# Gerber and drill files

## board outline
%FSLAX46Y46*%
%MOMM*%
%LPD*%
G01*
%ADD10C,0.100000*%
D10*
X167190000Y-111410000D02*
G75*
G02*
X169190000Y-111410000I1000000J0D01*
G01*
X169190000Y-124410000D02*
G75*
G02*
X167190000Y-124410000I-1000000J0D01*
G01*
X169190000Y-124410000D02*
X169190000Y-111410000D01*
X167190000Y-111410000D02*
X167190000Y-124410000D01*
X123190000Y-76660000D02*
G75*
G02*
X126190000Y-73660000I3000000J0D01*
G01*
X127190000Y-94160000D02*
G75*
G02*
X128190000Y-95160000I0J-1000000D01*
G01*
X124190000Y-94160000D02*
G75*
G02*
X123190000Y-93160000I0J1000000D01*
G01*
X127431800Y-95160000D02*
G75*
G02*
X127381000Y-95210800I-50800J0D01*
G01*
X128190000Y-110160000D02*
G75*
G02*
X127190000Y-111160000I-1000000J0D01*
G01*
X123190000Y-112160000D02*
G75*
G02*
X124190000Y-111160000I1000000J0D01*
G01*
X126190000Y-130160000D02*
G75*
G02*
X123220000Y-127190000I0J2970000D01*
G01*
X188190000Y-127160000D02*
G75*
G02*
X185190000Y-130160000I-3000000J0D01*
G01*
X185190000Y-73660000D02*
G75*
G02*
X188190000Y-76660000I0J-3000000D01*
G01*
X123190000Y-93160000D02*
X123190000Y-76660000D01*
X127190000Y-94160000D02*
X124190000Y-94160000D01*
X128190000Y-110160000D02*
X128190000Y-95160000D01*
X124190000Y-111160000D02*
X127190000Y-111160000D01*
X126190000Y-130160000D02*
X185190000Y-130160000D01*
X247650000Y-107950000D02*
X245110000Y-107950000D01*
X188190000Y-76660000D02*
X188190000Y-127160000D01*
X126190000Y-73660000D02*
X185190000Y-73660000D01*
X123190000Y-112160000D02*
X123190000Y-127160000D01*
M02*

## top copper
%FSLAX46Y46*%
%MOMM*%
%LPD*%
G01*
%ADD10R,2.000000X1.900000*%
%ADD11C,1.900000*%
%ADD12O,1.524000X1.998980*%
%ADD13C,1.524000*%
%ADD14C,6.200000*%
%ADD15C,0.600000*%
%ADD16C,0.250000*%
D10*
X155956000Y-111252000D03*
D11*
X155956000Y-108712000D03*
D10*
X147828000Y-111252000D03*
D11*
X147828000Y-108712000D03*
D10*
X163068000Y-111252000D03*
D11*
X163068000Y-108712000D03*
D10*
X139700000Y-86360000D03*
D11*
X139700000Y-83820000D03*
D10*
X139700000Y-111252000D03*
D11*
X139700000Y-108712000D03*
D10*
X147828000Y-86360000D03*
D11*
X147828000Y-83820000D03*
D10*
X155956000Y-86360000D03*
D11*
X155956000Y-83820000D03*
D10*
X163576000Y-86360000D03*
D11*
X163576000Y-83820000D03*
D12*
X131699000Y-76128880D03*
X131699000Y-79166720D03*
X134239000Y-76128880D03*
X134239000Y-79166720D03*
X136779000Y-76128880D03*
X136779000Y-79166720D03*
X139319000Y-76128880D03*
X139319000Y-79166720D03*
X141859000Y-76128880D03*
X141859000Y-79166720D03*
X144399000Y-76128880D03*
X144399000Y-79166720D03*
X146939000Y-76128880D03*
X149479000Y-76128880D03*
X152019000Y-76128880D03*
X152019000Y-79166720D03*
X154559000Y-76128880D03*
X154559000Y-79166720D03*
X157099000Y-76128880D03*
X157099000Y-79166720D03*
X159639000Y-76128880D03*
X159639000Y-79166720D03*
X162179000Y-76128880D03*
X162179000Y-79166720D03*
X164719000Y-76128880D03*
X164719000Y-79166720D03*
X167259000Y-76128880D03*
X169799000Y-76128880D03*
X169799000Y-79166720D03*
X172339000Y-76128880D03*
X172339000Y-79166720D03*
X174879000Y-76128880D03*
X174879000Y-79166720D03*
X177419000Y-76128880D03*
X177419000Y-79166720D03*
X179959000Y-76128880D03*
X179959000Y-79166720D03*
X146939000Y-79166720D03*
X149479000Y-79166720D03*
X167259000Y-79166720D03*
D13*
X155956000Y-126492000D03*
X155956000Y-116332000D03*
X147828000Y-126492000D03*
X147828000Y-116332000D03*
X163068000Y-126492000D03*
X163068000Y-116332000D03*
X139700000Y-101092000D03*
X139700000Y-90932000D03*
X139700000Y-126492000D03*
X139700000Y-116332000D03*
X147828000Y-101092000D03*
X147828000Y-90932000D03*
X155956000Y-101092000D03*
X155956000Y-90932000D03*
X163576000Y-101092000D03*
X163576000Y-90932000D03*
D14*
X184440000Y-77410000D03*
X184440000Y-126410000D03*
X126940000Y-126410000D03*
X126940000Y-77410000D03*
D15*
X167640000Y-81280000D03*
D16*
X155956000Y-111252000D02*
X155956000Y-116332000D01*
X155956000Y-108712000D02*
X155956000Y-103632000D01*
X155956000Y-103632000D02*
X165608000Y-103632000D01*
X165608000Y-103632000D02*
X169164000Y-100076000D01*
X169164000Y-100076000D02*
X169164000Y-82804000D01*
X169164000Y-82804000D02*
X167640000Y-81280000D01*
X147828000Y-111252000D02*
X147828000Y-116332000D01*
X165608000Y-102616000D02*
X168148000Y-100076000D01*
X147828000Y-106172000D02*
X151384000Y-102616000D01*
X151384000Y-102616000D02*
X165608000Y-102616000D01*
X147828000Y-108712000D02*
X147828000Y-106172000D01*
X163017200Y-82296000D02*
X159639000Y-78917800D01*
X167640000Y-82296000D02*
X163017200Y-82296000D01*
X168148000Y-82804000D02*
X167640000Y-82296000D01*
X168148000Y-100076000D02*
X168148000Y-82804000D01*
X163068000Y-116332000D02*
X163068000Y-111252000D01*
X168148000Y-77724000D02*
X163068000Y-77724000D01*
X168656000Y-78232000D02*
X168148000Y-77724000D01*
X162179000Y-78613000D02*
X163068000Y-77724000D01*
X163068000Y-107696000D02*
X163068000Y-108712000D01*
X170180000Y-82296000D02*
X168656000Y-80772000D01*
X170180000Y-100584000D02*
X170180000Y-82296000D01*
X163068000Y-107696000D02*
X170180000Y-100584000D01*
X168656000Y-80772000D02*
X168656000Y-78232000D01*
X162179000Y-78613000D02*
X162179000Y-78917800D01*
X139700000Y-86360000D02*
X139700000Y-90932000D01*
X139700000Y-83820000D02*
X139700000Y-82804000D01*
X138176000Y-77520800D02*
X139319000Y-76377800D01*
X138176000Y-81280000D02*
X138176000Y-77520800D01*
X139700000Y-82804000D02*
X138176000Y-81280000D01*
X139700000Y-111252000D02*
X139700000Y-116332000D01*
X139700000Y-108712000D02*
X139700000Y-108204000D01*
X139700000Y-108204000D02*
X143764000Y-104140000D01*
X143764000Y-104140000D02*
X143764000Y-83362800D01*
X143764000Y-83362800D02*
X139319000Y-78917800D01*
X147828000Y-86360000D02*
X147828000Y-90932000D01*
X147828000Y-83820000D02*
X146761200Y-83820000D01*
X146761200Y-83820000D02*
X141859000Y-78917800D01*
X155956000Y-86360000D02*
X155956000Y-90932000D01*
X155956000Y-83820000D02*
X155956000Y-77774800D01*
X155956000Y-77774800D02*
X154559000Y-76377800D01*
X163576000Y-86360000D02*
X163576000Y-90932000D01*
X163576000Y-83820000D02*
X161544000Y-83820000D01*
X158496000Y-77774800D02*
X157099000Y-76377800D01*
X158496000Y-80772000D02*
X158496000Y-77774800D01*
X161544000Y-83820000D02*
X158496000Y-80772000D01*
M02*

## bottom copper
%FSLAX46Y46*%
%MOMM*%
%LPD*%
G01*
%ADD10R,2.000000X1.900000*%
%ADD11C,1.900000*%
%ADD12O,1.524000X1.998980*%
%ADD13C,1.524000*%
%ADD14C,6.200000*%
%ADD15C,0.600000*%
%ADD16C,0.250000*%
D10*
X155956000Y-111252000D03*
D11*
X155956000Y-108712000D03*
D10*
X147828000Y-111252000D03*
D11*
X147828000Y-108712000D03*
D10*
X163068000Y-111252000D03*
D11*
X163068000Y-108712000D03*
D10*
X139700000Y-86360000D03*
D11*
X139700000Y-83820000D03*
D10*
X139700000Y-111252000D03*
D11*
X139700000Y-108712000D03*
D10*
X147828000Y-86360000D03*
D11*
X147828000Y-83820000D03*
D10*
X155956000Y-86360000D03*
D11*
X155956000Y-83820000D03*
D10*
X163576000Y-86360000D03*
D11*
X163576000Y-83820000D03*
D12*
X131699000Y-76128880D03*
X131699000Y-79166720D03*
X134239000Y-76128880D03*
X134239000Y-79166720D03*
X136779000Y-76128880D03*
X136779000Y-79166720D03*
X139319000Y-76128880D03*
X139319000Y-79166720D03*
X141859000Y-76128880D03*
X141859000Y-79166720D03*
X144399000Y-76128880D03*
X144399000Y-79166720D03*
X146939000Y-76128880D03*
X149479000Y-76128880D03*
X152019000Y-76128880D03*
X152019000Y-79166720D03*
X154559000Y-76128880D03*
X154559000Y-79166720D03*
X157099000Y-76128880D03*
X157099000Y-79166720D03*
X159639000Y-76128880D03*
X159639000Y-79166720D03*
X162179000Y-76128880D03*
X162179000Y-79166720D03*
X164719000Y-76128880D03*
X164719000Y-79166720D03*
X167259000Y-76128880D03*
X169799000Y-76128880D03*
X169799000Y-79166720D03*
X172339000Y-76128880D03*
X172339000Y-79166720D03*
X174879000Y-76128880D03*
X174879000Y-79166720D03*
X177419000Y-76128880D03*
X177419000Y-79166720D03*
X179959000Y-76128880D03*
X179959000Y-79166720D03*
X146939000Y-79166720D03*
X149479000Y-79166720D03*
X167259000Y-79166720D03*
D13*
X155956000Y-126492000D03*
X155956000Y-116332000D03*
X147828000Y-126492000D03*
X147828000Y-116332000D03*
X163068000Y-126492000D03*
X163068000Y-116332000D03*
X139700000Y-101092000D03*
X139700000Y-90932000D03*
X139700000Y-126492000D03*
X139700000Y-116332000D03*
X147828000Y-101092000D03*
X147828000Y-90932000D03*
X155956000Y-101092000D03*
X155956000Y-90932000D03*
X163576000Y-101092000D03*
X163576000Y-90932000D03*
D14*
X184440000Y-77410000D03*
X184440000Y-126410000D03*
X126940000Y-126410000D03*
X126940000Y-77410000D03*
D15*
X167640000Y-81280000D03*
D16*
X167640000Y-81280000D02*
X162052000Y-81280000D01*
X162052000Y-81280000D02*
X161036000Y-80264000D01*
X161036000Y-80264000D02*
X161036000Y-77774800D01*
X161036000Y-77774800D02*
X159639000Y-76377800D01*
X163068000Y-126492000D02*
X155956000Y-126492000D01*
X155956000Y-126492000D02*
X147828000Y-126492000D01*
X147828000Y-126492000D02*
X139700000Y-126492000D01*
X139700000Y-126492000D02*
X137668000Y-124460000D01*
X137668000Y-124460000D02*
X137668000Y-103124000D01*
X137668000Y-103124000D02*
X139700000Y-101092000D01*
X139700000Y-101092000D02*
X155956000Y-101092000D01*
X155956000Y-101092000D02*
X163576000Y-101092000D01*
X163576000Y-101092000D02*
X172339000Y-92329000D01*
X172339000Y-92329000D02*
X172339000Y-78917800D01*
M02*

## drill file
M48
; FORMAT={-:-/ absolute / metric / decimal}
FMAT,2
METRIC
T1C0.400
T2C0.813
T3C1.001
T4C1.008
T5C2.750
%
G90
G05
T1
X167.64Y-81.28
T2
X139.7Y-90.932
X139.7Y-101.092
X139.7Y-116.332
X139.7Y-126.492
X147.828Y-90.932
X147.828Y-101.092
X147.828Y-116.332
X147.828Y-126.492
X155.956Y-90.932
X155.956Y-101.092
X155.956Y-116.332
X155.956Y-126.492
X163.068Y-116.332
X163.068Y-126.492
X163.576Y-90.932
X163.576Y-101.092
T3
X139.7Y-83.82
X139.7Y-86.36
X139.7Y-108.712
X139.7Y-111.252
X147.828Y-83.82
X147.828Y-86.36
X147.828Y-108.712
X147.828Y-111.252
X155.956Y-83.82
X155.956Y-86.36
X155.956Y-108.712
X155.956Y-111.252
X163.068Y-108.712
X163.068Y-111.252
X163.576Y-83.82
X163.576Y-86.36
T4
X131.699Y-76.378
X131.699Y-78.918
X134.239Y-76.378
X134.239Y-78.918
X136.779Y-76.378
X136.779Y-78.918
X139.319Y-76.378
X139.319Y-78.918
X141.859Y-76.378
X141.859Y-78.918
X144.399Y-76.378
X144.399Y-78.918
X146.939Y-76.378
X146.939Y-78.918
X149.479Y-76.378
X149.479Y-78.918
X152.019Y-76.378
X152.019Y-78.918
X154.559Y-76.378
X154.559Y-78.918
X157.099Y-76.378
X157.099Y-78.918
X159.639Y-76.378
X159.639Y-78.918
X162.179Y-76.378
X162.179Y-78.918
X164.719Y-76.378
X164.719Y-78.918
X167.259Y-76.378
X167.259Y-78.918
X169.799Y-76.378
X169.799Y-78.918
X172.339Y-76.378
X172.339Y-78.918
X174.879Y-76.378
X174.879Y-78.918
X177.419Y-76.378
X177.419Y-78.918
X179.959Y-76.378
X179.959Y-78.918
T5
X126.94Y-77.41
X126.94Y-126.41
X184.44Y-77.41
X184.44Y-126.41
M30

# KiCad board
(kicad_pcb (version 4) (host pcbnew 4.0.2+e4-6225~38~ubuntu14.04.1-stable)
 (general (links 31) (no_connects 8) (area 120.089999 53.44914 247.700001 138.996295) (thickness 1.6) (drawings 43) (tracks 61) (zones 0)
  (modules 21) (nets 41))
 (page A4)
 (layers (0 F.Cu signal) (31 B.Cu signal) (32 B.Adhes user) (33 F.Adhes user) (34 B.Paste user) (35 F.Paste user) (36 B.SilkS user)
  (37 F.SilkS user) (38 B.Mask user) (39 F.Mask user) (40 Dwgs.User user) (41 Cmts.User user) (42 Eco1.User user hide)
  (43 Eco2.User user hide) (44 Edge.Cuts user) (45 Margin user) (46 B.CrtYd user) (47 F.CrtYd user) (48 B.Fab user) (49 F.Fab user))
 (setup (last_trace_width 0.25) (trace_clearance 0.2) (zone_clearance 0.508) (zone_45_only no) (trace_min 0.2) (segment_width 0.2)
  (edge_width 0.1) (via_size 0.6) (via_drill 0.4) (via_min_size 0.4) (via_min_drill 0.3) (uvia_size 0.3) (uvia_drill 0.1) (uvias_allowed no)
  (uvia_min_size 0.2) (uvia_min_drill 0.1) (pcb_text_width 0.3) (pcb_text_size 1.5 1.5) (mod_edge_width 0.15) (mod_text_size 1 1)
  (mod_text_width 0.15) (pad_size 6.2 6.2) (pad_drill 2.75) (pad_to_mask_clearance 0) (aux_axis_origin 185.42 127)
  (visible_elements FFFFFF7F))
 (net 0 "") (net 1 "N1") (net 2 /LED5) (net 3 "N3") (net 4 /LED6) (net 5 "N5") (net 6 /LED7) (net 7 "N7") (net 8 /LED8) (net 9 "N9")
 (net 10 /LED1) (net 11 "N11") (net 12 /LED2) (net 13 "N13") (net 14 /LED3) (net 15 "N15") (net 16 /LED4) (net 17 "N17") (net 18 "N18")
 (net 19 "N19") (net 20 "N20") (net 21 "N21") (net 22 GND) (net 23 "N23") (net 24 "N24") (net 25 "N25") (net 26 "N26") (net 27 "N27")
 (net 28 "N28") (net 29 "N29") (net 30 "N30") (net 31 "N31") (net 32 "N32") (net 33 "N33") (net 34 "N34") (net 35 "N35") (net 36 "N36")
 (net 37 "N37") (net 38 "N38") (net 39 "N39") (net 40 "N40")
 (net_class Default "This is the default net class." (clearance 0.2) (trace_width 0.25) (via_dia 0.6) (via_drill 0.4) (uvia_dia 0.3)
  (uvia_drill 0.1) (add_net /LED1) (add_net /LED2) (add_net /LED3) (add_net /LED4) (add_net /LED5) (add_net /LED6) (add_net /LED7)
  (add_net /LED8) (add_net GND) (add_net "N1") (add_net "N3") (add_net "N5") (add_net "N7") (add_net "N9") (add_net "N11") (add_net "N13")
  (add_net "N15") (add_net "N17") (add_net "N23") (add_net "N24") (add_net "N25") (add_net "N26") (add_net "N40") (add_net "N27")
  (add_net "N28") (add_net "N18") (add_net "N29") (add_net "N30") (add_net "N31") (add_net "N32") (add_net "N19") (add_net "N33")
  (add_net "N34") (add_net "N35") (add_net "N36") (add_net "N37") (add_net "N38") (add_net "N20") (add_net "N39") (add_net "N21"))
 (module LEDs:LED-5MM (layer F.Cu) (at 155.956 111.252 90)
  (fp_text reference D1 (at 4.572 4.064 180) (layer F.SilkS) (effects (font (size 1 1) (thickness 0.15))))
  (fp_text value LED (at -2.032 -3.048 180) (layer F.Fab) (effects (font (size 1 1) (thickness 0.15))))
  (pad 1 thru_hole rect (at 0 0 180) (size 2 1.9) (drill 1.00076) (layers *.Cu *.Mask F.SilkS) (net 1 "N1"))
  (pad 2 thru_hole circle (at 2.54 0 90) (size 1.9 1.9) (drill 1.00076) (layers *.Cu *.Mask F.SilkS) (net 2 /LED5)))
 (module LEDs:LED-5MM (layer F.Cu) (at 147.828 111.252 90)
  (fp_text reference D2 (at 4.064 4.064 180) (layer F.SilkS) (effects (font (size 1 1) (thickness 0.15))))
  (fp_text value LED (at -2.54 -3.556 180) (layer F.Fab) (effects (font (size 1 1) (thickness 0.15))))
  (pad 1 thru_hole rect (at 0 0 180) (size 2 1.9) (drill 1.00076) (layers *.Cu *.Mask F.SilkS) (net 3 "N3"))
  (pad 2 thru_hole circle (at 2.54 0 90) (size 1.9 1.9) (drill 1.00076) (layers *.Cu *.Mask F.SilkS) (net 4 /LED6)))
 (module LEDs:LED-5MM (layer F.Cu) (at 163.068 111.252 90)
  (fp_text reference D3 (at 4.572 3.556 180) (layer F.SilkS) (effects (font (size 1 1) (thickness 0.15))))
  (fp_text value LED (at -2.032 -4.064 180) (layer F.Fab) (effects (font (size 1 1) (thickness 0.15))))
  (pad 1 thru_hole rect (at 0 0 180) (size 2 1.9) (drill 1.00076) (layers *.Cu *.Mask F.SilkS) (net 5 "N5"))
  (pad 2 thru_hole circle (at 2.54 0 90) (size 1.9 1.9) (drill 1.00076) (layers *.Cu *.Mask F.SilkS) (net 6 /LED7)))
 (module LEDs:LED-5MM (layer F.Cu) (at 139.7 86.36 90)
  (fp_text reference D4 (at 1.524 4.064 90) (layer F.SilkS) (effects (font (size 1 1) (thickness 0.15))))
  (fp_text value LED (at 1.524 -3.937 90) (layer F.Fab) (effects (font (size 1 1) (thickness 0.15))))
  (pad 1 thru_hole rect (at 0 0 180) (size 2 1.9) (drill 1.00076) (layers *.Cu *.Mask F.SilkS) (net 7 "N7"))
  (pad 2 thru_hole circle (at 2.54 0 90) (size 1.9 1.9) (drill 1.00076) (layers *.Cu *.Mask F.SilkS) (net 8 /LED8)))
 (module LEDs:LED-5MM (layer F.Cu) (at 139.7 111.252 90)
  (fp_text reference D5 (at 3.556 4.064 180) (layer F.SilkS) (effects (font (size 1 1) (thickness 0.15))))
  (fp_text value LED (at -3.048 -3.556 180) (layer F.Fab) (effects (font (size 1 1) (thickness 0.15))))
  (pad 1 thru_hole rect (at 0 0 180) (size 2 1.9) (drill 1.00076) (layers *.Cu *.Mask F.SilkS) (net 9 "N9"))
  (pad 2 thru_hole circle (at 2.54 0 90) (size 1.9 1.9) (drill 1.00076) (layers *.Cu *.Mask F.SilkS) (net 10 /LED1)))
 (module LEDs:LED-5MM (layer F.Cu) (at 147.828 86.36 90)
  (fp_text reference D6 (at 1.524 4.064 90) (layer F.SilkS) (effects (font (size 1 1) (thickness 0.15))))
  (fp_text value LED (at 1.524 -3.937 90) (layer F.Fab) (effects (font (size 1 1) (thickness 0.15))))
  (pad 1 thru_hole rect (at 0 0 180) (size 2 1.9) (drill 1.00076) (layers *.Cu *.Mask F.SilkS) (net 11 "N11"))
  (pad 2 thru_hole circle (at 2.54 0 90) (size 1.9 1.9) (drill 1.00076) (layers *.Cu *.Mask F.SilkS) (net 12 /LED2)))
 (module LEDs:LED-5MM (layer F.Cu) (at 155.956 86.36 90)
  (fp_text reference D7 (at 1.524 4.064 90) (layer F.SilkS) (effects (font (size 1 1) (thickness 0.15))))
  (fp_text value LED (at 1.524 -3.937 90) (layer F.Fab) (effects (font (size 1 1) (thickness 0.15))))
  (pad 1 thru_hole rect (at 0 0 180) (size 2 1.9) (drill 1.00076) (layers *.Cu *.Mask F.SilkS) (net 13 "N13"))
  (pad 2 thru_hole circle (at 2.54 0 90) (size 1.9 1.9) (drill 1.00076) (layers *.Cu *.Mask F.SilkS) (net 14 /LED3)))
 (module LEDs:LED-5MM (layer F.Cu) (at 163.576 86.36 90)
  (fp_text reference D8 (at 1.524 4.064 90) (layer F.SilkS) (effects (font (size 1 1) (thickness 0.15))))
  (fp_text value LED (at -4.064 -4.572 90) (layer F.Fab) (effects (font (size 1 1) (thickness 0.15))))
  (pad 1 thru_hole rect (at 0 0 180) (size 2 1.9) (drill 1.00076) (layers *.Cu *.Mask F.SilkS) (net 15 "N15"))
  (pad 2 thru_hole circle (at 2.54 0 90) (size 1.9 1.9) (drill 1.00076) (layers *.Cu *.Mask F.SilkS) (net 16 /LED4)))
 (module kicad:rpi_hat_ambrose (layer F.Cu) (at 155.829 80.1878)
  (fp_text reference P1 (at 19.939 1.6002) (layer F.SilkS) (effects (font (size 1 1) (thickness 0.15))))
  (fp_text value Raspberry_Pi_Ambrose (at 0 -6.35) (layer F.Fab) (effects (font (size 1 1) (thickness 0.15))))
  (pad 1 thru_hole oval (at -24.13 -3.81) (size 1.524 1.99898) (drill 1.0076 (offset 0 -0.24892)) (layers *.Cu *.Mask F.SilkS)
   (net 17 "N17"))
  (pad 2 thru_hole oval (at -24.13 -1.27) (size 1.524 1.99898) (drill 1.0076 (offset 0 0.24892)) (layers *.Cu *.Mask F.SilkS) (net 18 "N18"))
  (pad 3 thru_hole oval (at -21.59 -3.81) (size 1.524 1.99898) (drill 1.0076 (offset 0 -0.24892)) (layers *.Cu *.Mask F.SilkS)
   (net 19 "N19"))
  (pad 4 thru_hole oval (at -21.59 -1.27) (size 1.524 1.99898) (drill 1.0076 (offset 0 0.24892)) (layers *.Cu *.Mask F.SilkS) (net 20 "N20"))
  (pad 5 thru_hole oval (at -19.05 -3.81) (size 1.524 1.99898) (drill 1.0076 (offset 0 -0.24892)) (layers *.Cu *.Mask F.SilkS)
   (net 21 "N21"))
  (pad 6 thru_hole oval (at -19.05 -1.27) (size 1.524 1.99898) (drill 1.0076 (offset 0 0.24892)) (layers *.Cu *.Mask F.SilkS) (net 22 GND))
  (pad 7 thru_hole oval (at -16.51 -3.81) (size 1.524 1.99898) (drill 1.0076 (offset 0 -0.24892)) (layers *.Cu *.Mask F.SilkS) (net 8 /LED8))
  (pad 8 thru_hole oval (at -16.51 -1.27) (size 1.524 1.99898) (drill 1.0076 (offset 0 0.24892)) (layers *.Cu *.Mask F.SilkS) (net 10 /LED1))
  (pad 9 thru_hole oval (at -13.97 -3.81) (size 1.524 1.99898) (drill 1.0076 (offset 0 -0.24892)) (layers *.Cu *.Mask F.SilkS) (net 22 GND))
  (pad 10 thru_hole oval (at -13.97 -1.27) (size 1.524 1.99898) (drill 1.0076 (offset 0 0.24892)) (layers *.Cu *.Mask F.SilkS)
   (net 12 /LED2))
  (pad 11 thru_hole oval (at -11.43 -3.81) (size 1.524 1.99898) (drill 1.0076 (offset 0 -0.24892)) (layers *.Cu *.Mask F.SilkS)
   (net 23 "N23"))
  (pad 12 thru_hole oval (at -11.43 -1.27) (size 1.524 1.99898) (drill 1.0076 (offset 0 0.24892)) (layers *.Cu *.Mask F.SilkS)
   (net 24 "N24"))
  (pad 13 thru_hole oval (at -8.89 -3.81) (size 1.524 1.99898) (drill 1.0076 (offset 0 -0.24892)) (layers *.Cu *.Mask F.SilkS)
   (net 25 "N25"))
  (pad 15 thru_hole oval (at -6.35 -3.81) (size 1.524 1.99898) (drill 1.0076 (offset 0 -0.24892)) (layers *.Cu *.Mask F.SilkS)
   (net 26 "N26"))
  (pad 17 thru_hole oval (at -3.81 -3.81) (size 1.524 1.99898) (drill 1.0076 (offset 0 -0.24892)) (layers *.Cu *.Mask F.SilkS)
   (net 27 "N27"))
  (pad 18 thru_hole oval (at -3.81 -1.27) (size 1.524 1.99898) (drill 1.0076 (offset 0 0.24892)) (layers *.Cu *.Mask F.SilkS) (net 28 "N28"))
  (pad 19 thru_hole oval (at -1.27 -3.81) (size 1.524 1.99898) (drill 1.0076 (offset 0 -0.24892)) (layers *.Cu *.Mask F.SilkS)
   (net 14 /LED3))
  (pad 20 thru_hole oval (at -1.27 -1.27) (size 1.524 1.99898) (drill 1.0076 (offset 0 0.24892)) (layers *.Cu *.Mask F.SilkS) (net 22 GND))
  (pad 21 thru_hole oval (at 1.27 -3.81) (size 1.524 1.99898) (drill 1.0076 (offset 0 -0.24892)) (layers *.Cu *.Mask F.SilkS) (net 16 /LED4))
  (pad 22 thru_hole oval (at 1.27 -1.27) (size 1.524 1.99898) (drill 1.0076 (offset 0 0.24892)) (layers *.Cu *.Mask F.SilkS) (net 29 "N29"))
  (pad 23 thru_hole oval (at 3.81 -3.81) (size 1.524 1.99898) (drill 1.0076 (offset 0 -0.24892)) (layers *.Cu *.Mask F.SilkS) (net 2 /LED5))
  (pad 24 thru_hole oval (at 3.81 -1.27) (size 1.524 1.99898) (drill 1.0076 (offset 0 0.24892)) (layers *.Cu *.Mask F.SilkS) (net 4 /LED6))
  (pad 25 thru_hole oval (at 6.35 -3.81) (size 1.524 1.99898) (drill 1.0076 (offset 0 -0.24892)) (layers *.Cu *.Mask F.SilkS) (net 22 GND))
  (pad 26 thru_hole oval (at 6.35 -1.27) (size 1.524 1.99898) (drill 1.0076 (offset 0 0.24892)) (layers *.Cu *.Mask F.SilkS) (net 6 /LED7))
  (pad 27 thru_hole oval (at 8.89 -3.81) (size 1.524 1.99898) (drill 1.0076 (offset 0 -0.24892)) (layers *.Cu *.Mask F.SilkS) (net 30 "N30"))
  (pad 28 thru_hole oval (at 8.89 -1.27) (size 1.524 1.99898) (drill 1.0076 (offset 0 0.24892)) (layers *.Cu *.Mask F.SilkS) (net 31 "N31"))
  (pad 29 thru_hole oval (at 11.43 -3.81) (size 1.524 1.99898) (drill 1.0076 (offset 0 -0.24892)) (layers *.Cu *.Mask F.SilkS)
   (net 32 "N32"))
  (pad 31 thru_hole oval (at 13.97 -3.81) (size 1.524 1.99898) (drill 1.0076 (offset 0 -0.24892)) (layers *.Cu *.Mask F.SilkS)
   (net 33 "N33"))
  (pad 32 thru_hole oval (at 13.97 -1.27) (size 1.524 1.99898) (drill 1.0076 (offset 0 0.24892)) (layers *.Cu *.Mask F.SilkS) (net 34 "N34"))
  (pad 33 thru_hole oval (at 16.51 -3.81) (size 1.524 1.99898) (drill 1.0076 (offset 0 -0.24892)) (layers *.Cu *.Mask F.SilkS)
   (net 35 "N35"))
  (pad 34 thru_hole oval (at 16.51 -1.27) (size 1.524 1.99898) (drill 1.0076 (offset 0 0.24892)) (layers *.Cu *.Mask F.SilkS) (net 22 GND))
  (pad 35 thru_hole oval (at 19.05 -3.81) (size 1.524 1.99898) (drill 1.0076 (offset 0 -0.24892)) (layers *.Cu *.Mask F.SilkS)
   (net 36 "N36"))
  (pad 36 thru_hole oval (at 19.05 -1.27) (size 1.524 1.99898) (drill 1.0076 (offset 0 0.24892)) (layers *.Cu *.Mask F.SilkS) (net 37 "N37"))
  (pad 37 thru_hole oval (at 21.59 -3.81) (size 1.524 1.99898) (drill 1.0076 (offset 0 -0.24892)) (layers *.Cu *.Mask F.SilkS)
   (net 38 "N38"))
  (pad 38 thru_hole oval (at 21.59 -1.27) (size 1.524 1.99898) (drill 1.0076 (offset 0 0.24892)) (layers *.Cu *.Mask F.SilkS))
  (pad 39 thru_hole oval (at 24.13 -3.81) (size 1.524 1.99898) (drill 1.0076 (offset 0 -0.24892)) (layers *.Cu *.Mask F.SilkS) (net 22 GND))
  (pad 40 thru_hole oval (at 24.13 -1.27) (size 1.524 1.99898) (drill 1.0076 (offset 0 0.24892)) (layers *.Cu *.Mask F.SilkS) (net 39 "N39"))
  (pad 14 thru_hole oval (at -8.89 -1.27) (size 1.524 1.99898) (drill 1.0076 (offset 0 0.24892)) (layers *.Cu *.Mask F.SilkS) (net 22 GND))
  (pad 16 thru_hole oval (at -6.35 -1.27) (size 1.524 1.99898) (drill 1.0076 (offset 0 0.24892)) (layers *.Cu *.Mask F.SilkS) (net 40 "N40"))
  (pad 30 thru_hole oval (at 11.43 -1.27) (size 1.524 1.99898) (drill 1.0076 (offset 0 0.24892)) (layers *.Cu *.Mask F.SilkS) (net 22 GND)))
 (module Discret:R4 (layer F.Cu) (at 155.956 121.412 90)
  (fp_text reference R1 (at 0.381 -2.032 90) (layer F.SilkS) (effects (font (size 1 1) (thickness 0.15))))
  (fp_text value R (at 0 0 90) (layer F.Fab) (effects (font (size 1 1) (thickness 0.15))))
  (pad 1 thru_hole circle (at -5.08 0 90) (size 1.524 1.524) (drill 0.8128) (layers *.Cu *.Mask F.SilkS) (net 22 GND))
  (pad 2 thru_hole circle (at 5.08 0 90) (size 1.524 1.524) (drill 0.8128) (layers *.Cu *.Mask F.SilkS) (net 1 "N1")))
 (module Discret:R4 (layer F.Cu) (at 147.828 121.412 90)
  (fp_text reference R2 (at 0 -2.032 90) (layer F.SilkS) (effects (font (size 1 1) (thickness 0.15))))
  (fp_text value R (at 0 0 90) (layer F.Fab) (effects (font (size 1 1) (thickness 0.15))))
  (pad 1 thru_hole circle (at -5.08 0 90) (size 1.524 1.524) (drill 0.8128) (layers *.Cu *.Mask F.SilkS) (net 22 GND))
  (pad 2 thru_hole circle (at 5.08 0 90) (size 1.524 1.524) (drill 0.8128) (layers *.Cu *.Mask F.SilkS) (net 3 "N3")))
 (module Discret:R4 (layer F.Cu) (at 163.068 121.412 90)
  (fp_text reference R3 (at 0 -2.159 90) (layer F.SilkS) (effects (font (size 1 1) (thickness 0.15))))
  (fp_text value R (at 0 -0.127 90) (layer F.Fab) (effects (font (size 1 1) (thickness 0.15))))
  (pad 1 thru_hole circle (at -5.08 0 90) (size 1.524 1.524) (drill 0.8128) (layers *.Cu *.Mask F.SilkS) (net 22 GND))
  (pad 2 thru_hole circle (at 5.08 0 90) (size 1.524 1.524) (drill 0.8128) (layers *.Cu *.Mask F.SilkS) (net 5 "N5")))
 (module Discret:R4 (layer F.Cu) (at 139.7 96.012 90)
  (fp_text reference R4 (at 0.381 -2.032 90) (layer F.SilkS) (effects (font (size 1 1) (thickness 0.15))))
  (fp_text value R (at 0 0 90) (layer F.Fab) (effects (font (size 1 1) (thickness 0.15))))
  (pad 1 thru_hole circle (at -5.08 0 90) (size 1.524 1.524) (drill 0.8128) (layers *.Cu *.Mask F.SilkS) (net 22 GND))
  (pad 2 thru_hole circle (at 5.08 0 90) (size 1.524 1.524) (drill 0.8128) (layers *.Cu *.Mask F.SilkS) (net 7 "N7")))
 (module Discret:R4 (layer F.Cu) (at 139.7 121.412 90)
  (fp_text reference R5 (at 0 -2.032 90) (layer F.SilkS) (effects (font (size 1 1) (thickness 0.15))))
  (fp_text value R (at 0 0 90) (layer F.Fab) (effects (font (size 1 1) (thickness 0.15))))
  (pad 1 thru_hole circle (at -5.08 0 90) (size 1.524 1.524) (drill 0.8128) (layers *.Cu *.Mask F.SilkS) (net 22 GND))
  (pad 2 thru_hole circle (at 5.08 0 90) (size 1.524 1.524) (drill 0.8128) (layers *.Cu *.Mask F.SilkS) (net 9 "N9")))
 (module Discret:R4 (layer F.Cu) (at 147.828 96.012 90)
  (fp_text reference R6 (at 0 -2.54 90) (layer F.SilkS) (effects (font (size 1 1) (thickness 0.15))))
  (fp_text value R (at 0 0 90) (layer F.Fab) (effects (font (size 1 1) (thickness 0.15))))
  (pad 1 thru_hole circle (at -5.08 0 90) (size 1.524 1.524) (drill 0.8128) (layers *.Cu *.Mask F.SilkS) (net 22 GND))
  (pad 2 thru_hole circle (at 5.08 0 90) (size 1.524 1.524) (drill 0.8128) (layers *.Cu *.Mask F.SilkS) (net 11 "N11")))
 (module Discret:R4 (layer F.Cu) (at 155.956 96.012 90)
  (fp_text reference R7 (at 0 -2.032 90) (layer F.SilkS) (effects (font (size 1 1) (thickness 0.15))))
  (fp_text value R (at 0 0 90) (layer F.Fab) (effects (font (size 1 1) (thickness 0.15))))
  (pad 1 thru_hole circle (at -5.08 0 90) (size 1.524 1.524) (drill 0.8128) (layers *.Cu *.Mask F.SilkS) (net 22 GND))
  (pad 2 thru_hole circle (at 5.08 0 90) (size 1.524 1.524) (drill 0.8128) (layers *.Cu *.Mask F.SilkS) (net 13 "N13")))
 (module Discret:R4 (layer F.Cu) (at 163.576 96.012 90)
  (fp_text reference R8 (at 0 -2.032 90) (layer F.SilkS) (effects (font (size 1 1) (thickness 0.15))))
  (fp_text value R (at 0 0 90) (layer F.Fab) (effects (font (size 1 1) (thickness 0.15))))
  (pad 1 thru_hole circle (at -5.08 0 90) (size 1.524 1.524) (drill 0.8128) (layers *.Cu *.Mask F.SilkS) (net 22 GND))
  (pad 2 thru_hole circle (at 5.08 0 90) (size 1.524 1.524) (drill 0.8128) (layers *.Cu *.Mask F.SilkS) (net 15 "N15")))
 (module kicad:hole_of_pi (layer F.Cu) (at 184.658 77.216)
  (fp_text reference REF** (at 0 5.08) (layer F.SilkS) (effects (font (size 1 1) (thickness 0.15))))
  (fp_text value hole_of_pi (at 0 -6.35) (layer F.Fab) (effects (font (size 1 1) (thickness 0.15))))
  (pad 1 thru_hole circle (at -0.218 0.194) (size 6.2 6.2) (drill 2.75) (layers *.Cu *.Mask F.SilkS)))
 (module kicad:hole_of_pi (layer F.Cu) (at 184.531 126.492)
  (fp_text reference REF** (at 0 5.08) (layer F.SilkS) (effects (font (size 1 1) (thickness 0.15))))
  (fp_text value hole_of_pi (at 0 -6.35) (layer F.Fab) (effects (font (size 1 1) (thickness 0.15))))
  (pad 1 thru_hole circle (at -0.091 -0.082) (size 6.2 6.2) (drill 2.75) (layers *.Cu *.Mask F.SilkS)))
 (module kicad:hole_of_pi (layer F.Cu) (at 126.873 126.492)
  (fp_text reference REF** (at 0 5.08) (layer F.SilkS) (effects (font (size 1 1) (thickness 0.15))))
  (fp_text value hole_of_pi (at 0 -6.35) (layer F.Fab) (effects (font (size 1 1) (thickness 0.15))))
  (pad 1 thru_hole circle (at 0.067 -0.082) (size 6.2 6.2) (drill 2.75) (layers *.Cu *.Mask F.SilkS)))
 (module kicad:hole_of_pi (layer F.Cu) (at 126.746 77.597)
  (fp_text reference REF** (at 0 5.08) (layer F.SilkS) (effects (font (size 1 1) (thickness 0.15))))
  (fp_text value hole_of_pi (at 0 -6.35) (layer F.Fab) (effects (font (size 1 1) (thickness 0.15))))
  (pad 1 thru_hole circle (at 0.194 -0.187) (size 6.2 6.2) (drill 2.75) (layers *.Cu *.Mask F.SilkS)))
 (gr_arc (start 168.19 111.41) (end 167.19 111.41) (angle 180) (layer Edge.Cuts) (width 0.1))
 (gr_arc (start 168.19 124.41) (end 169.19 124.41) (angle 180) (layer Edge.Cuts) (width 0.1))
 (gr_line (start 169.19 124.41) (end 169.19 111.41) (angle 90) (layer Edge.Cuts) (width 0.1))
 (gr_line (start 167.19 111.41) (end 167.19 124.41) (angle 90) (layer Edge.Cuts) (width 0.1))
 (gr_arc (start 126.19 76.66) (end 123.19 76.66) (angle 90) (layer Edge.Cuts) (width 0.1))
 (gr_arc (start 127.19 95.16) (end 127.19 94.16) (angle 90) (layer Edge.Cuts) (width 0.1))
 (gr_arc (start 124.19 93.16) (end 124.19 94.16) (angle 90) (layer Edge.Cuts) (width 0.1))
 (gr_arc (start 127.381 95.16) (end 127.4318 95.16) (angle 90) (layer Edge.Cuts) (width 0.1))
 (gr_arc (start 127.19 110.16) (end 128.19 110.16) (angle 90) (layer Edge.Cuts) (width 0.1))
 (gr_arc (start 124.19 112.16) (end 123.19 112.16) (angle 90) (layer Edge.Cuts) (width 0.1))
 (gr_arc (start 126.19 127.19) (end 126.19 130.16) (angle 90) (layer Edge.Cuts) (width 0.1))
 (gr_arc (start 185.19 127.16) (end 188.19 127.16) (angle 90) (layer Edge.Cuts) (width 0.1))
 (gr_arc (start 185.19 76.66) (end 185.19 73.66) (angle 90) (layer Edge.Cuts) (width 0.1))
 (gr_line (start 123.19 93.16) (end 123.19 76.66) (angle 90) (layer Edge.Cuts) (width 0.1))
 (gr_line (start 127.19 94.16) (end 124.19 94.16) (angle 90) (layer Edge.Cuts) (width 0.1))
 (gr_line (start 128.19 110.16) (end 128.19 95.16) (angle 90) (layer Edge.Cuts) (width 0.1))
 (gr_line (start 124.19 111.16) (end 127.19 111.16) (angle 90) (layer Edge.Cuts) (width 0.1))
 (gr_line (start 126.19 130.16) (end 185.19 130.16) (angle 90) (layer Edge.Cuts) (width 0.1))
 (gr_line (start 247.65 107.95) (end 245.11 107.95) (angle 90) (layer Edge.Cuts) (width 0.1))
 (gr_line (start 188.19 76.66) (end 188.19 127.16) (angle 90) (layer Edge.Cuts) (width 0.1))
 (gr_line (start 126.19 73.66) (end 185.19 73.66) (angle 90) (layer Edge.Cuts) (width 0.1))
 (gr_line (start 123.19 112.16) (end 123.19 127.16) (angle 90) (layer Edge.Cuts) (width 0.1))
 (segment (start 155.956 111.252) (end 155.956 116.332) (width 0.25) (layer F.Cu) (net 1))
 (segment (start 155.956 108.712) (end 155.956 103.632) (width 0.25) (layer F.Cu) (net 2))
 (segment (start 155.956 103.632) (end 165.608 103.632) (width 0.25) (layer F.Cu) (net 2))
 (segment (start 165.608 103.632) (end 169.164 100.076) (width 0.25) (layer F.Cu) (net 2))
 (segment (start 169.164 100.076) (end 169.164 82.804) (width 0.25) (layer F.Cu) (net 2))
 (segment (start 169.164 82.804) (end 167.64 81.28) (width 0.25) (layer F.Cu) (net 2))
 (via (at 167.64 81.28) (size 0.6) (drill 0.4) (layers F.Cu B.Cu) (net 2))
 (segment (start 167.64 81.28) (end 162.052 81.28) (width 0.25) (layer B.Cu) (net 2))
 (segment (start 162.052 81.28) (end 161.036 80.264) (width 0.25) (layer B.Cu) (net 2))
 (segment (start 161.036 80.264) (end 161.036 77.7748) (width 0.25) (layer B.Cu) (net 2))
 (segment (start 161.036 77.7748) (end 159.639 76.3778) (width 0.25) (layer B.Cu) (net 2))
 (segment (start 147.828 111.252) (end 147.828 116.332) (width 0.25) (layer F.Cu) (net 3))
 (segment (start 165.608 102.616) (end 168.148 100.076) (width 0.25) (layer F.Cu) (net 4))
 (segment (start 147.828 106.172) (end 151.384 102.616) (width 0.25) (layer F.Cu) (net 4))
 (segment (start 151.384 102.616) (end 165.608 102.616) (width 0.25) (layer F.Cu) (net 4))
 (segment (start 147.828 108.712) (end 147.828 106.172) (width 0.25) (layer F.Cu) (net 4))
 (segment (start 163.0172 82.296) (end 159.639 78.9178) (width 0.25) (layer F.Cu) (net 4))
 (segment (start 167.64 82.296) (end 163.0172 82.296) (width 0.25) (layer F.Cu) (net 4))
 (segment (start 168.148 82.804) (end 167.64 82.296) (width 0.25) (layer F.Cu) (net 4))
 (segment (start 168.148 100.076) (end 168.148 82.804) (width 0.25) (layer F.Cu) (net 4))
 (segment (start 163.068 116.332) (end 163.068 111.252) (width 0.25) (layer F.Cu) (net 5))
 (segment (start 168.148 77.724) (end 163.068 77.724) (width 0.25) (layer F.Cu) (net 6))
 (segment (start 168.656 78.232) (end 168.148 77.724) (width 0.25) (layer F.Cu) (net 6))
 (segment (start 162.179 78.613) (end 163.068 77.724) (width 0.25) (layer F.Cu) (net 6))
 (segment (start 163.068 107.696) (end 163.068 108.712) (width 0.25) (layer F.Cu) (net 6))
 (segment (start 170.18 82.296) (end 168.656 80.772) (width 0.25) (layer F.Cu) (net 6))
 (segment (start 170.18 100.584) (end 170.18 82.296) (width 0.25) (layer F.Cu) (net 6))
 (segment (start 163.068 107.696) (end 170.18 100.584) (width 0.25) (layer F.Cu) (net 6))
 (segment (start 168.656 80.772) (end 168.656 78.232) (width 0.25) (layer F.Cu) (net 6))
 (segment (start 162.179 78.613) (end 162.179 78.9178) (width 0.25) (layer F.Cu) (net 6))
 (segment (start 139.7 86.36) (end 139.7 90.932) (width 0.25) (layer F.Cu) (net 7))
 (segment (start 139.7 83.82) (end 139.7 82.804) (width 0.25) (layer F.Cu) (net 8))
 (segment (start 138.176 77.5208) (end 139.319 76.3778) (width 0.25) (layer F.Cu) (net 8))
 (segment (start 138.176 81.28) (end 138.176 77.5208) (width 0.25) (layer F.Cu) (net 8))
 (segment (start 139.7 82.804) (end 138.176 81.28) (width 0.25) (layer F.Cu) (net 8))
 (segment (start 139.7 111.252) (end 139.7 116.332) (width 0.25) (layer F.Cu) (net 9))
 (segment (start 139.7 108.712) (end 139.7 108.204) (width 0.25) (layer F.Cu) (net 10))
 (segment (start 139.7 108.204) (end 143.764 104.14) (width 0.25) (layer F.Cu) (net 10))
 (segment (start 143.764 104.14) (end 143.764 83.3628) (width 0.25) (layer F.Cu) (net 10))
 (segment (start 143.764 83.3628) (end 139.319 78.9178) (width 0.25) (layer F.Cu) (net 10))
 (segment (start 147.828 86.36) (end 147.828 90.932) (width 0.25) (layer F.Cu) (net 11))
 (segment (start 147.828 83.82) (end 146.7612 83.82) (width 0.25) (layer F.Cu) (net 12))
 (segment (start 146.7612 83.82) (end 141.859 78.9178) (width 0.25) (layer F.Cu) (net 12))
 (segment (start 155.956 86.36) (end 155.956 90.932) (width 0.25) (layer F.Cu) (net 13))
 (segment (start 155.956 83.82) (end 155.956 77.7748) (width 0.25) (layer F.Cu) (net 14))
 (segment (start 155.956 77.7748) (end 154.559 76.3778) (width 0.25) (layer F.Cu) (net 14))
 (segment (start 163.576 86.36) (end 163.576 90.932) (width 0.25) (layer F.Cu) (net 15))
 (segment (start 163.576 83.82) (end 161.544 83.82) (width 0.25) (layer F.Cu) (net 16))
 (segment (start 158.496 77.7748) (end 157.099 76.3778) (width 0.25) (layer F.Cu) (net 16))
 (segment (start 158.496 80.772) (end 158.496 77.7748) (width 0.25) (layer F.Cu) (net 16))
 (segment (start 161.544 83.82) (end 158.496 80.772) (width 0.25) (layer F.Cu) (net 16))
 (segment (start 163.068 126.492) (end 155.956 126.492) (width 0.25) (layer B.Cu) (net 22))
 (segment (start 155.956 126.492) (end 147.828 126.492) (width 0.25) (layer B.Cu) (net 22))
 (segment (start 147.828 126.492) (end 139.7 126.492) (width 0.25) (layer B.Cu) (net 22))
 (segment (start 139.7 126.492) (end 137.668 124.46) (width 0.25) (layer B.Cu) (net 22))
 (segment (start 137.668 124.46) (end 137.668 103.124) (width 0.25) (layer B.Cu) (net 22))
 (segment (start 137.668 103.124) (end 139.7 101.092) (width 0.25) (layer B.Cu) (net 22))
 (segment (start 139.7 101.092) (end 155.956 101.092) (width 0.25) (layer B.Cu) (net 22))
 (segment (start 155.956 101.092) (end 163.576 101.092) (width 0.25) (layer B.Cu) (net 22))
 (segment (start 163.576 101.092) (end 172.339 92.329) (width 0.25) (layer B.Cu) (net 22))
 (segment (start 172.339 92.329) (end 172.339 78.9178) (width 0.25) (layer B.Cu) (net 22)))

